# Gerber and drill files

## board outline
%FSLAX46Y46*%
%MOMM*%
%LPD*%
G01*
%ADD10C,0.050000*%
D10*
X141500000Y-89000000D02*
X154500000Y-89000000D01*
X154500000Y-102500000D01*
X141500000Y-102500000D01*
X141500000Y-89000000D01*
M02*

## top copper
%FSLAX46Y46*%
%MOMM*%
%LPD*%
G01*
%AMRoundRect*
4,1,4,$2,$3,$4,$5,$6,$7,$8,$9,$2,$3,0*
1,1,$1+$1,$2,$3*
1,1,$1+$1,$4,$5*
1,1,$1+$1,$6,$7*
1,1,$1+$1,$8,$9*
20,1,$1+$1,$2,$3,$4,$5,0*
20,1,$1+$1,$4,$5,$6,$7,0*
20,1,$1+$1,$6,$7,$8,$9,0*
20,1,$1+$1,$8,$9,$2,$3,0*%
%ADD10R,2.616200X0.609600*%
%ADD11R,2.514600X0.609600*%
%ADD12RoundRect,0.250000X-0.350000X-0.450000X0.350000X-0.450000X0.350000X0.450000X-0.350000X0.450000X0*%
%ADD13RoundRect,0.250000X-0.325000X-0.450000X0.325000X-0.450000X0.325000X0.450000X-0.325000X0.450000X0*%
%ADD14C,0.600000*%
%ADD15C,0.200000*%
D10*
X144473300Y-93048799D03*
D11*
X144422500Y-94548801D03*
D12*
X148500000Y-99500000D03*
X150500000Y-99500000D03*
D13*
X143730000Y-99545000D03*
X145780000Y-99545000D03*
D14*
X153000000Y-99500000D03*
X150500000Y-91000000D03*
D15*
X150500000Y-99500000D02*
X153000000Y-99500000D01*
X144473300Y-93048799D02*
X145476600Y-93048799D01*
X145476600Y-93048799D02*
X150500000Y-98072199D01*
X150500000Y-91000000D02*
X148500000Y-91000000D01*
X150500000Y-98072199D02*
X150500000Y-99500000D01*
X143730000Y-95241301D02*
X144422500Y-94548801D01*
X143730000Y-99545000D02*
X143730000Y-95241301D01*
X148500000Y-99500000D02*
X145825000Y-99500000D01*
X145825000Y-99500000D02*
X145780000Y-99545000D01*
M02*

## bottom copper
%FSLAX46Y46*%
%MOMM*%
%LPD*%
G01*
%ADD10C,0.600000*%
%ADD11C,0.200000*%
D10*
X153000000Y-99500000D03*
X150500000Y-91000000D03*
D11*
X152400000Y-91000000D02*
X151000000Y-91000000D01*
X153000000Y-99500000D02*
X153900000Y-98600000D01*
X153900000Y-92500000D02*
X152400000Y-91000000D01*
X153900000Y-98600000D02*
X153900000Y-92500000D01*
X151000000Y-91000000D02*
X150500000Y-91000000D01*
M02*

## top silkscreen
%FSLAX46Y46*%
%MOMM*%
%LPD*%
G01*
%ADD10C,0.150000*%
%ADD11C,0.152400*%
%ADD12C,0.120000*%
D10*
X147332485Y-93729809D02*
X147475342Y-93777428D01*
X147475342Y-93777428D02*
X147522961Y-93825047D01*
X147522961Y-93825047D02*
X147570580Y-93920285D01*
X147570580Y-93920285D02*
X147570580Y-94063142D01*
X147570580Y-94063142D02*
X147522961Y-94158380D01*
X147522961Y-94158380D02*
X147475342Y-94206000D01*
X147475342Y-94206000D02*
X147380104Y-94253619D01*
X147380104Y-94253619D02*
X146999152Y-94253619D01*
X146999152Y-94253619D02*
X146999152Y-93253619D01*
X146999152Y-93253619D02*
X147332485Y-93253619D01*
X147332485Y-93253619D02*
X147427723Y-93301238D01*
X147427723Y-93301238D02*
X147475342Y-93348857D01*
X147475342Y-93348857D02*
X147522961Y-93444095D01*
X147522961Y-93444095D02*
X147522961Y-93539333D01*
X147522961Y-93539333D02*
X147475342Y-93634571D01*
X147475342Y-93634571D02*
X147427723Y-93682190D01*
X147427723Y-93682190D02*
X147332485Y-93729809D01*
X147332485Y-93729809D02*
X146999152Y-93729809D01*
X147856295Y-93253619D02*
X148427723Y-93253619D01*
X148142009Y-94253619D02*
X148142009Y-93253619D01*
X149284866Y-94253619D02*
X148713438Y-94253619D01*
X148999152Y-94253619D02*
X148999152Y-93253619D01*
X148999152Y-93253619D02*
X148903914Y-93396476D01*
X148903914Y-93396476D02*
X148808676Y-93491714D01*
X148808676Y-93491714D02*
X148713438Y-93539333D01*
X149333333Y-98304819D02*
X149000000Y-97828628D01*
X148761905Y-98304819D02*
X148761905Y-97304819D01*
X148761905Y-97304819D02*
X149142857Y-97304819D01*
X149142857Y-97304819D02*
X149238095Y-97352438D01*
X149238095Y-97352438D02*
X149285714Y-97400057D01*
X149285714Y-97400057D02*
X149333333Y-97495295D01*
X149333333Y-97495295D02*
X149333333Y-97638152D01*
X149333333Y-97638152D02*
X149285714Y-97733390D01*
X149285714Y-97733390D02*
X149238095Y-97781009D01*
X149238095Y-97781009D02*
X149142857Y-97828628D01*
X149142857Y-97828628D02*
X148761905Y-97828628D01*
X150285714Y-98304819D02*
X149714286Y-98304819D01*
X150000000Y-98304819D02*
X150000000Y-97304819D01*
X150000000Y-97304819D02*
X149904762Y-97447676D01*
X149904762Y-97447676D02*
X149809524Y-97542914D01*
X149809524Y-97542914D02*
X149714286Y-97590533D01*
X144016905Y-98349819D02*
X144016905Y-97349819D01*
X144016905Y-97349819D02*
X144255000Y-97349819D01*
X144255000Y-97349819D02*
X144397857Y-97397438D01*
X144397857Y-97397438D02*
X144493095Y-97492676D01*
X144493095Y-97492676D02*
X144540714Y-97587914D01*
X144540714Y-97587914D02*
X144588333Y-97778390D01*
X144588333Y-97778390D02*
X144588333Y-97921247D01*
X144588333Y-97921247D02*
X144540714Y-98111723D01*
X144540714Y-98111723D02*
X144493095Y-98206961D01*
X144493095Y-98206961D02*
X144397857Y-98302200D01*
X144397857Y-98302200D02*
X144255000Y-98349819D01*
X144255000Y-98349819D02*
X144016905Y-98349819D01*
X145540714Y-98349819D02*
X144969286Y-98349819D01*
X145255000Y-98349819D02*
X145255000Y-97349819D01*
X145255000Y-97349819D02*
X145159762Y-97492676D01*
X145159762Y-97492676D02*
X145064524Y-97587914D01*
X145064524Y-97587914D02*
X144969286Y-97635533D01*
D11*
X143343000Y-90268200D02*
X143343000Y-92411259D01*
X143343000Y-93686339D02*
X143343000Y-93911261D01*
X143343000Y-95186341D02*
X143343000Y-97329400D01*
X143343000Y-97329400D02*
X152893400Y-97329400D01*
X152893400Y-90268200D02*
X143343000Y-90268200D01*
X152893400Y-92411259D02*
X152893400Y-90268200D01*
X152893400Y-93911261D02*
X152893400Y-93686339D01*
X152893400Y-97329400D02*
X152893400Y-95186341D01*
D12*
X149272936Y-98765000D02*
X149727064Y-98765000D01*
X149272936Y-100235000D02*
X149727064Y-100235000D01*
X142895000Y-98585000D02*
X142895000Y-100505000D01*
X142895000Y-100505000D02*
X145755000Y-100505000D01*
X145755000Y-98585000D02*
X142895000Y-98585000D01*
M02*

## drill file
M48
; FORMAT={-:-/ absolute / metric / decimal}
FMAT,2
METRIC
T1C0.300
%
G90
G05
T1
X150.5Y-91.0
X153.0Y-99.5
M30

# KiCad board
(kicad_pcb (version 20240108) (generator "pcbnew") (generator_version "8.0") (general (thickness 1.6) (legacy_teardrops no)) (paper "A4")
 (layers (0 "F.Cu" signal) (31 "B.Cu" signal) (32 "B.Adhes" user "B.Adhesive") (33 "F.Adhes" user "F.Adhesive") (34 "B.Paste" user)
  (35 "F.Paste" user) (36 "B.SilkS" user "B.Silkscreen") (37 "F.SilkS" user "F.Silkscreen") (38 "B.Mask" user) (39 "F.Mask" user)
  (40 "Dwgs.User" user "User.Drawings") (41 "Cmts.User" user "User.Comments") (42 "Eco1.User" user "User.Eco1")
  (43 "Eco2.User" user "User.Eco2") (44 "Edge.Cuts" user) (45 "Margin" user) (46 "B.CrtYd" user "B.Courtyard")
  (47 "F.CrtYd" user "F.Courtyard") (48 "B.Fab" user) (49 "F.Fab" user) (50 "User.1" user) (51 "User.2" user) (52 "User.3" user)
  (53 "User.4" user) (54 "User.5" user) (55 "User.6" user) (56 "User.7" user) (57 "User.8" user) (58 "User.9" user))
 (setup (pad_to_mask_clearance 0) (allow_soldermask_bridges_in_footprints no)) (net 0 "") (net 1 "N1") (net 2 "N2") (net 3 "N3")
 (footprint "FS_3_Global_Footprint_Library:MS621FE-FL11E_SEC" (layer "F.Cu") (at 148.1182 93.7988)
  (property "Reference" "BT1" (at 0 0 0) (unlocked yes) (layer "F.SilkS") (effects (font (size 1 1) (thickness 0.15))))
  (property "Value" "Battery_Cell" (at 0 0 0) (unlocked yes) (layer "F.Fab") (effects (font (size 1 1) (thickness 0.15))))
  (fp_line (start -4.7752 -3.5306) (end -4.7752 -1.387541) (stroke (width 0.1524) (type solid)) (layer "F.SilkS"))
  (fp_line (start -4.7752 -0.112461) (end -4.7752 0.112461) (stroke (width 0.1524) (type solid)) (layer "F.SilkS"))
  (fp_line (start -4.7752 1.387541) (end -4.7752 3.5306) (stroke (width 0.1524) (type solid)) (layer "F.SilkS"))
  (fp_line (start -4.7752 3.5306) (end 4.7752 3.5306) (stroke (width 0.1524) (type solid)) (layer "F.SilkS"))
  (fp_line (start 4.7752 -3.5306) (end -4.7752 -3.5306) (stroke (width 0.1524) (type solid)) (layer "F.SilkS"))
  (fp_line (start 4.7752 -1.387541) (end 4.7752 -3.5306) (stroke (width 0.1524) (type solid)) (layer "F.SilkS"))
  (fp_line (start 4.7752 0.112461) (end 4.7752 -0.112461) (stroke (width 0.1524) (type solid)) (layer "F.SilkS"))
  (fp_line (start 4.7752 3.5306) (end 4.7752 1.387541) (stroke (width 0.1524) (type solid)) (layer "F.SilkS"))
  (pad "1" smd rect (at -3.6449 -0.750001) (size 2.6162 0.6096) (layers "F.Cu" "F.Paste" "F.Mask") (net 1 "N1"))
  (pad "2" smd rect (at -3.6957 0.750001) (size 2.5146 0.6096) (layers "F.Cu" "F.Paste" "F.Mask") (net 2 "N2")))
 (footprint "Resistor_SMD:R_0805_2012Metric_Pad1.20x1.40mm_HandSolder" (layer "F.Cu") (at 149.5 99.5)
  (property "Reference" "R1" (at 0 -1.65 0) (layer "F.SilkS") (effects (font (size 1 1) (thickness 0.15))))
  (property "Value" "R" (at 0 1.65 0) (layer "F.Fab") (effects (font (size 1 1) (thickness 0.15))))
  (fp_line (start -0.227064 -0.735) (end 0.227064 -0.735) (stroke (width 0.12) (type solid)) (layer "F.SilkS"))
  (fp_line (start -0.227064 0.735) (end 0.227064 0.735) (stroke (width 0.12) (type solid)) (layer "F.SilkS"))
  (pad "1" smd roundrect (at -1 0) (size 1.2 1.4) (layers "F.Cu" "F.Paste" "F.Mask") (roundrect_rratio 0.208333) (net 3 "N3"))
  (pad "2" smd roundrect (at 1 0) (size 1.2 1.4) (layers "F.Cu" "F.Paste" "F.Mask") (roundrect_rratio 0.208333) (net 1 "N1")))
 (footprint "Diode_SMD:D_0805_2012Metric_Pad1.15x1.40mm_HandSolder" (layer "F.Cu") (at 144.755 99.545)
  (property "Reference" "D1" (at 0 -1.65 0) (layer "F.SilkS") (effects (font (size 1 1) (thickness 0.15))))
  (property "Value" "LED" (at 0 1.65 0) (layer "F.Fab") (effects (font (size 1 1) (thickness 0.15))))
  (fp_line (start -1.86 -0.96) (end -1.86 0.96) (stroke (width 0.12) (type solid)) (layer "F.SilkS"))
  (fp_line (start -1.86 0.96) (end 1 0.96) (stroke (width 0.12) (type solid)) (layer "F.SilkS"))
  (fp_line (start 1 -0.96) (end -1.86 -0.96) (stroke (width 0.12) (type solid)) (layer "F.SilkS"))
  (pad "1" smd roundrect (at -1.025 0) (size 1.15 1.4) (layers "F.Cu" "F.Paste" "F.Mask") (roundrect_rratio 0.217391) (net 2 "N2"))
  (pad "2" smd roundrect (at 1.025 0) (size 1.15 1.4) (layers "F.Cu" "F.Paste" "F.Mask") (roundrect_rratio 0.217391) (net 3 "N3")))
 (gr_rect (start 141.5 89) (end 154.5 102.5) (stroke (width 0.05) (type default)) (fill none) (layer "Edge.Cuts"))
 (segment (start 150.5 99.5) (end 153 99.5) (width 0.2) (layer "F.Cu") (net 1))
 (segment (start 144.4733 93.048799) (end 145.4766 93.048799) (width 0.2) (layer "F.Cu") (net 1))
 (segment (start 145.4766 93.048799) (end 150.5 98.072199) (width 0.2) (layer "F.Cu") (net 1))
 (segment (start 150.5 91) (end 148.5 91) (width 0.2) (layer "F.Cu") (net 1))
 (segment (start 150.5 98.072199) (end 150.5 99.5) (width 0.2) (layer "F.Cu") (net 1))
 (via (at 153 99.5) (size 0.6) (drill 0.3) (layers "F.Cu" "B.Cu") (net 1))
 (via (at 150.5 91) (size 0.6) (drill 0.3) (layers "F.Cu" "B.Cu") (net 1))
 (segment (start 152.4 91) (end 151 91) (width 0.2) (layer "B.Cu") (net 1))
 (segment (start 153 99.5) (end 153.9 98.6) (width 0.2) (layer "B.Cu") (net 1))
 (segment (start 153.9 92.5) (end 152.4 91) (width 0.2) (layer "B.Cu") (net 1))
 (segment (start 153.9 98.6) (end 153.9 92.5) (width 0.2) (layer "B.Cu") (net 1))
 (segment (start 151 91) (end 150.5 91) (width 0.2) (layer "B.Cu") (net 1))
 (segment (start 143.73 95.241301) (end 144.4225 94.548801) (width 0.2) (layer "F.Cu") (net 2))
 (segment (start 143.73 99.545) (end 143.73 95.241301) (width 0.2) (layer "F.Cu") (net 2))
 (segment (start 148.5 99.5) (end 145.825 99.5) (width 0.2) (layer "F.Cu") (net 3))
 (segment (start 145.825 99.5) (end 145.78 99.545) (width 0.2) (layer "F.Cu") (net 3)))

